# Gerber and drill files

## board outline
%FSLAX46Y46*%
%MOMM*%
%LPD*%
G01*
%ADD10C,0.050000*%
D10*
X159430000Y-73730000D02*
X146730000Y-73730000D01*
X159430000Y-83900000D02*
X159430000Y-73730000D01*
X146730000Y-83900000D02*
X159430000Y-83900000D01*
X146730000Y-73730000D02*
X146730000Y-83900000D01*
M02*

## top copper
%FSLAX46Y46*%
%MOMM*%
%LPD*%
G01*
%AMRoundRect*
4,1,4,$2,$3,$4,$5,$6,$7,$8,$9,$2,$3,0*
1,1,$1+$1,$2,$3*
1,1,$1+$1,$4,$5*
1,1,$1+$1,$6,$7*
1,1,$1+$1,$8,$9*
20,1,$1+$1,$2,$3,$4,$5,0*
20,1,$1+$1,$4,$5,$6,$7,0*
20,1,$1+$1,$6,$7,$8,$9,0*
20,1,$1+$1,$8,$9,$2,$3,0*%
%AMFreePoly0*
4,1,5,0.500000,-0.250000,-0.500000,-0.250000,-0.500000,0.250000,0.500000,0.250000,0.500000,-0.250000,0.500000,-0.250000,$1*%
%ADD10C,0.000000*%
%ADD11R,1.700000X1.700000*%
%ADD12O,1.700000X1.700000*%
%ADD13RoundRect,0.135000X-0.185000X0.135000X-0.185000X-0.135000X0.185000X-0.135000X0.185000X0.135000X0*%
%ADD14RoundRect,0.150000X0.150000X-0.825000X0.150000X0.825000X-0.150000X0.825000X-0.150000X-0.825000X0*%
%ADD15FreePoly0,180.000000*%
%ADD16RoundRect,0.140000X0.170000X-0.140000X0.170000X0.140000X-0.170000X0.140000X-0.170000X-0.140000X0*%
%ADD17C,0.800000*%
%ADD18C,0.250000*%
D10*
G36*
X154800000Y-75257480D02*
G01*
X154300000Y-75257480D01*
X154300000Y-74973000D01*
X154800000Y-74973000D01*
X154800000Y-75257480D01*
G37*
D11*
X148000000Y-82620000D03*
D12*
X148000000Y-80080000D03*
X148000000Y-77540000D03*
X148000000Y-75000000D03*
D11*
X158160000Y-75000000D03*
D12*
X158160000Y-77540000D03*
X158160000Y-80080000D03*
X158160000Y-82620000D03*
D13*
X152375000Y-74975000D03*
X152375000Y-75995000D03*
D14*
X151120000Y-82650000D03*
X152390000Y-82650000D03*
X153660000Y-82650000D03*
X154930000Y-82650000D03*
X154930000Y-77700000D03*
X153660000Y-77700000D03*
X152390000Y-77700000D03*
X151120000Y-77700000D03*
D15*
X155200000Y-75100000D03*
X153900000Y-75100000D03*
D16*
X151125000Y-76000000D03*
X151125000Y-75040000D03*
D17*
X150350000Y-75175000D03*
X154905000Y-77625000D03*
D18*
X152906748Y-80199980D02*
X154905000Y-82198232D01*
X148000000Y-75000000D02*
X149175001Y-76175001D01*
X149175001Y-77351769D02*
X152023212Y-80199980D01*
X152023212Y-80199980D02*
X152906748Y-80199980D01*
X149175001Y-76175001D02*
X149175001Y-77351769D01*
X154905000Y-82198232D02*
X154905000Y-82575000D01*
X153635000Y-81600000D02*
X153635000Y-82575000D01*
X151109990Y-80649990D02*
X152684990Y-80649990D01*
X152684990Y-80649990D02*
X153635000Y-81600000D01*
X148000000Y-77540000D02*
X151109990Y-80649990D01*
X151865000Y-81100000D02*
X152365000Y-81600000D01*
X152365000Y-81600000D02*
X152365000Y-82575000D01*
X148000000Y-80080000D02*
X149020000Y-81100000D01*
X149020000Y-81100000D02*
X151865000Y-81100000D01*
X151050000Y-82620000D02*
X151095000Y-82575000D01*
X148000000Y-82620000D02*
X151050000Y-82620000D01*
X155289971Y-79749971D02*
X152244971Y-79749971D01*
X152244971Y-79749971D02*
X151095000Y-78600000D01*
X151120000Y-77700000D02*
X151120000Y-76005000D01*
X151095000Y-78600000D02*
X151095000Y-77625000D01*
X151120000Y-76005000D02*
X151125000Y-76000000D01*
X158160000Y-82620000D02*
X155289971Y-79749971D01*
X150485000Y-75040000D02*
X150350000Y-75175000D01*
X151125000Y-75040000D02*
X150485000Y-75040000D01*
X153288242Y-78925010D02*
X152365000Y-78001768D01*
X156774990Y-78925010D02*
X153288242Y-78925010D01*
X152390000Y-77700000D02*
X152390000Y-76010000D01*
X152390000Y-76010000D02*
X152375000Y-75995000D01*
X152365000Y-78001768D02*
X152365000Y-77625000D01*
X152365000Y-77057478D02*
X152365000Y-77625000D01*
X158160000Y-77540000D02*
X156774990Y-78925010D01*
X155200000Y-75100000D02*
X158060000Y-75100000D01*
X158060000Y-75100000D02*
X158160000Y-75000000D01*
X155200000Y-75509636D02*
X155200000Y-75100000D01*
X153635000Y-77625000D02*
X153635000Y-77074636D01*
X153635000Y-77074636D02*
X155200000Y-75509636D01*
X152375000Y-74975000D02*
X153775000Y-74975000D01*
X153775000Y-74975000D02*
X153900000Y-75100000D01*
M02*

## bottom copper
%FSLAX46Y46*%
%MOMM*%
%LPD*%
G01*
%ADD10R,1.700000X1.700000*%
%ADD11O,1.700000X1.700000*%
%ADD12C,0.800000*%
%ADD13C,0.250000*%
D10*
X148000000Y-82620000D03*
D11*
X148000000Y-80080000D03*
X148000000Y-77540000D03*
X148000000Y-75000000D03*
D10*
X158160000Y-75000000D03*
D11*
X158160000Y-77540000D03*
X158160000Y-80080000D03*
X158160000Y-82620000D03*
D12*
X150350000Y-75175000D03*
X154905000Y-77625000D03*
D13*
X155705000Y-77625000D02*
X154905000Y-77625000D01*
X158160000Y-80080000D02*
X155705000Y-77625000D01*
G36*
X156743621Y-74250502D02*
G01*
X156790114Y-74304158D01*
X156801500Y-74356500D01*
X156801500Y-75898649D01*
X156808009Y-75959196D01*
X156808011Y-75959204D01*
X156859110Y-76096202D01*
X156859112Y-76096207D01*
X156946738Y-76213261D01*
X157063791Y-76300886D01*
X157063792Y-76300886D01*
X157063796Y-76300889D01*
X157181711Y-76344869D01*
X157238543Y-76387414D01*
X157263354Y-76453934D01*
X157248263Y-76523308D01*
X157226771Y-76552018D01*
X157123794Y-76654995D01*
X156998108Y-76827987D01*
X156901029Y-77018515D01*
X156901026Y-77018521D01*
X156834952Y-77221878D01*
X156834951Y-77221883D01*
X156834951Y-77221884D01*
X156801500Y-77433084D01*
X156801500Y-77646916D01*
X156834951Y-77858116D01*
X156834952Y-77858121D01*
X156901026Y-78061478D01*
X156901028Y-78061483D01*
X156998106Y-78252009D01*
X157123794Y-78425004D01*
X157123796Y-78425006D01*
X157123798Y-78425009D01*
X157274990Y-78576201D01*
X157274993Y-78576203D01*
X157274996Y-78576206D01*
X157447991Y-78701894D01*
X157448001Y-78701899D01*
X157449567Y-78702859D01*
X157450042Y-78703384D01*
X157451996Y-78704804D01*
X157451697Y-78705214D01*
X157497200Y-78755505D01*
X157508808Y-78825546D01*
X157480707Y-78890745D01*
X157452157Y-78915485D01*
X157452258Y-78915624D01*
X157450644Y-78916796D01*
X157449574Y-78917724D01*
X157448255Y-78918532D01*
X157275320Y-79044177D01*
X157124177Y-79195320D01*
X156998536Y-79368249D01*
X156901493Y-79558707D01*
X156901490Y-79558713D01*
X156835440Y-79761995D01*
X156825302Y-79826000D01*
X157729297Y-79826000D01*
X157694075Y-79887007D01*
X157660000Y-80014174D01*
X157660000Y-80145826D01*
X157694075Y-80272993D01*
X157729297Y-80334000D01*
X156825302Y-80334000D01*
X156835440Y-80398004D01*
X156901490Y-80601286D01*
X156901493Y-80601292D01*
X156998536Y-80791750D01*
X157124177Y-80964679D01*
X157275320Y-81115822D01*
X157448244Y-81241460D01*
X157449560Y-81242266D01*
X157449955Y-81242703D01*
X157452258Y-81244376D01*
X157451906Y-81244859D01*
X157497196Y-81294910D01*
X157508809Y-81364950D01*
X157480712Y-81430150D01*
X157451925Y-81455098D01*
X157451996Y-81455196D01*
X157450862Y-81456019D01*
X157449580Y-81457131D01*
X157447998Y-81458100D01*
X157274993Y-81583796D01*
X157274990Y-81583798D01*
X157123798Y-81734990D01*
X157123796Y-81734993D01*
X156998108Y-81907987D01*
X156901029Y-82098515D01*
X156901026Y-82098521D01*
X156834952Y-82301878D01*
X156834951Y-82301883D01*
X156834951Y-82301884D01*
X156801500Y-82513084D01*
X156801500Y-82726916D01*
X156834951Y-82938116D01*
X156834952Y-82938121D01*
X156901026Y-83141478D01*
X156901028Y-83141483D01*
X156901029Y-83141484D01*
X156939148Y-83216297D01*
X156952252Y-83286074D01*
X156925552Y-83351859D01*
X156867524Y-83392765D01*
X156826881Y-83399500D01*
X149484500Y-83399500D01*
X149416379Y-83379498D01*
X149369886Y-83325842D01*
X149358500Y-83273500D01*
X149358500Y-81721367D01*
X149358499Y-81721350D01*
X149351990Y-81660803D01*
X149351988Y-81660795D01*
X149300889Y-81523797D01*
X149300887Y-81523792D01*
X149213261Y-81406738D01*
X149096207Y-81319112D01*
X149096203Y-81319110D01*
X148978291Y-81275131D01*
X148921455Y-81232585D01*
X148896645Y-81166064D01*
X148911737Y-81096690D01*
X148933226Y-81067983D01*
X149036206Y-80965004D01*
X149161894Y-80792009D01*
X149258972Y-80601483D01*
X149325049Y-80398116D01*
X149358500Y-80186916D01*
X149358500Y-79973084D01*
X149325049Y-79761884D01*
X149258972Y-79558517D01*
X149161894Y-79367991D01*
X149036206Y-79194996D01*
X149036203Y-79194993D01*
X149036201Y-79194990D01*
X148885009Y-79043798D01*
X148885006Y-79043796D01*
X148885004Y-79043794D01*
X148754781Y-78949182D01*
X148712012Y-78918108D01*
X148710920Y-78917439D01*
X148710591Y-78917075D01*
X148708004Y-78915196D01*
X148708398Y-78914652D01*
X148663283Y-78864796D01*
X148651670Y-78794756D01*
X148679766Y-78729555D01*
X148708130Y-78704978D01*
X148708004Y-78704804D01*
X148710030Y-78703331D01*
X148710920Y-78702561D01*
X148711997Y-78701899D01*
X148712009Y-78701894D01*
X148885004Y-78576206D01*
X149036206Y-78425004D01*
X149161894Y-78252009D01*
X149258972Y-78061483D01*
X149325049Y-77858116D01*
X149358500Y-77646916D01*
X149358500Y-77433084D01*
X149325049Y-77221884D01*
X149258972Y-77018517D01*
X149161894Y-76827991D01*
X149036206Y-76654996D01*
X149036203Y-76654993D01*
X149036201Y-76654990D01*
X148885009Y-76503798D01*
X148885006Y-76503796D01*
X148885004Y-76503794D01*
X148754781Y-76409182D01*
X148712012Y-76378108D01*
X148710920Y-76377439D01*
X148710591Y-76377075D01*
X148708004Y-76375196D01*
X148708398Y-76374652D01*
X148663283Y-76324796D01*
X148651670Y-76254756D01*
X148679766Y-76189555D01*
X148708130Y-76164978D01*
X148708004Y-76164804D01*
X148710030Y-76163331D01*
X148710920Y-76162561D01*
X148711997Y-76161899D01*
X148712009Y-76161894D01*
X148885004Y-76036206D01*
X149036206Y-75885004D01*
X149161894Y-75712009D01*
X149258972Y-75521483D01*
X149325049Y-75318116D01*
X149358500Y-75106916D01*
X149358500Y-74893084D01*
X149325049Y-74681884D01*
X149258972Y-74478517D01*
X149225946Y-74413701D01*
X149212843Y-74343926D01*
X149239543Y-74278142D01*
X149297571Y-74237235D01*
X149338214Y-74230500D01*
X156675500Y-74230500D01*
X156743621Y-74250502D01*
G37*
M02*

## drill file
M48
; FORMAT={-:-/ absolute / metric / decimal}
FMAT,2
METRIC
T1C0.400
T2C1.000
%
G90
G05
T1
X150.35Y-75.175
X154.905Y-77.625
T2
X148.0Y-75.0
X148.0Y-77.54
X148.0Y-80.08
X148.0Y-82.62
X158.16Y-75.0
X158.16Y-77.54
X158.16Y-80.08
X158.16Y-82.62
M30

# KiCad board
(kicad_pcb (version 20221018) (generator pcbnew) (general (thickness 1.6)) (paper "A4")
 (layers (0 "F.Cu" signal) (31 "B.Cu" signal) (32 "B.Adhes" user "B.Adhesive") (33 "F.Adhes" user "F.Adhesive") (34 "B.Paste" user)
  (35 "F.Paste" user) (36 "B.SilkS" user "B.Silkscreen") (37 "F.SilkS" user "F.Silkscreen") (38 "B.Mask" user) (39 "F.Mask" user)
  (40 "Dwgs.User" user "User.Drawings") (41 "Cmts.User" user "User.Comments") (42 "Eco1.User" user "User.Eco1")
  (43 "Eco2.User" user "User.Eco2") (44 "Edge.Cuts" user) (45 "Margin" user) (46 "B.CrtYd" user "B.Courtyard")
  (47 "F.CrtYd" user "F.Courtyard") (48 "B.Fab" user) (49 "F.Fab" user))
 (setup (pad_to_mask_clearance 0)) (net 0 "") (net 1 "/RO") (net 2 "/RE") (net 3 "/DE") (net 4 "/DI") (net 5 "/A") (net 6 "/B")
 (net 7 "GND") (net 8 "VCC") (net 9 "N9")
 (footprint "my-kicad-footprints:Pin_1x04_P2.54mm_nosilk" (layer "F.Cu") (at 148 82.62 180)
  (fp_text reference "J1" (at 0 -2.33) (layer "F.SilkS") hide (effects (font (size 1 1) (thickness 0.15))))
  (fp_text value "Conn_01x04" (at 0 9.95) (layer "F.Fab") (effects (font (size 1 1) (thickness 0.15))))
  (pad "1" thru_hole rect (at 0 0 180) (size 1.7 1.7) (drill 1) (layers "*.Cu" "*.Mask") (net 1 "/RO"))
  (pad "2" thru_hole oval (at 0 2.54 180) (size 1.7 1.7) (drill 1) (layers "*.Cu" "*.Mask") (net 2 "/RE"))
  (pad "3" thru_hole oval (at 0 5.08 180) (size 1.7 1.7) (drill 1) (layers "*.Cu" "*.Mask") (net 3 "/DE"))
  (pad "4" thru_hole oval (at 0 7.62 180) (size 1.7 1.7) (drill 1) (layers "*.Cu" "*.Mask") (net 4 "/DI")))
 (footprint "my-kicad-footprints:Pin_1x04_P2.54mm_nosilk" (layer "F.Cu") (at 158.16 75)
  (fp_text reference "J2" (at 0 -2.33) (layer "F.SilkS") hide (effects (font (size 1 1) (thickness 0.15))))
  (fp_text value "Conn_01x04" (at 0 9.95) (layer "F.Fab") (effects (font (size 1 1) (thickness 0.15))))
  (pad "1" thru_hole rect (at 0 0) (size 1.7 1.7) (drill 1) (layers "*.Cu" "*.Mask") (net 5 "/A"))
  (pad "2" thru_hole oval (at 0 2.54) (size 1.7 1.7) (drill 1) (layers "*.Cu" "*.Mask") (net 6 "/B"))
  (pad "3" thru_hole oval (at 0 5.08) (size 1.7 1.7) (drill 1) (layers "*.Cu" "*.Mask") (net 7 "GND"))
  (pad "4" thru_hole oval (at 0 7.62) (size 1.7 1.7) (drill 1) (layers "*.Cu" "*.Mask") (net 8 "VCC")))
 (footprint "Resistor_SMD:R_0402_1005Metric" (layer "F.Cu") (at 152.375 75.485 -90)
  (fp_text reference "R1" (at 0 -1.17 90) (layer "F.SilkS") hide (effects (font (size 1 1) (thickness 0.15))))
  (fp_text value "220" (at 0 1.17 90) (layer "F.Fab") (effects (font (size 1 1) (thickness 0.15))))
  (pad "1" smd roundrect (at -0.51 0 270) (size 0.54 0.64) (layers "F.Cu" "F.Paste" "F.Mask") (roundrect_rratio 0.25) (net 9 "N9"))
  (pad "2" smd roundrect (at 0.51 0 270) (size 0.54 0.64) (layers "F.Cu" "F.Paste" "F.Mask") (roundrect_rratio 0.25) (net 6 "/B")))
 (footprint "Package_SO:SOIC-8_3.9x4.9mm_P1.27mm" (layer "F.Cu") (at 153.025 80.175 90)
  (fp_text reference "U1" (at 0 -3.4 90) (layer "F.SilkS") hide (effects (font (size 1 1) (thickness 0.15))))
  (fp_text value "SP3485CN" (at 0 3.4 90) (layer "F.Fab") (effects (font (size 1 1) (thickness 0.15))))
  (pad "1" smd roundrect (at -2.475 -1.905 90) (size 1.95 0.6) (layers "F.Cu" "F.Paste" "F.Mask") (roundrect_rratio 0.25) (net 1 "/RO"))
  (pad "2" smd roundrect (at -2.475 -0.635 90) (size 1.95 0.6) (layers "F.Cu" "F.Paste" "F.Mask") (roundrect_rratio 0.25) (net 2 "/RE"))
  (pad "3" smd roundrect (at -2.475 0.635 90) (size 1.95 0.6) (layers "F.Cu" "F.Paste" "F.Mask") (roundrect_rratio 0.25) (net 3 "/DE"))
  (pad "4" smd roundrect (at -2.475 1.905 90) (size 1.95 0.6) (layers "F.Cu" "F.Paste" "F.Mask") (roundrect_rratio 0.25) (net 4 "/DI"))
  (pad "5" smd roundrect (at 2.475 1.905 90) (size 1.95 0.6) (layers "F.Cu" "F.Paste" "F.Mask") (roundrect_rratio 0.25) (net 7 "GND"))
  (pad "6" smd roundrect (at 2.475 0.635 90) (size 1.95 0.6) (layers "F.Cu" "F.Paste" "F.Mask") (roundrect_rratio 0.25) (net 5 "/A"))
  (pad "7" smd roundrect (at 2.475 -0.635 90) (size 1.95 0.6) (layers "F.Cu" "F.Paste" "F.Mask") (roundrect_rratio 0.25) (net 6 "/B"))
  (pad "8" smd roundrect (at 2.475 -1.905 90) (size 1.95 0.6) (layers "F.Cu" "F.Paste" "F.Mask") (roundrect_rratio 0.25) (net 8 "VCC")))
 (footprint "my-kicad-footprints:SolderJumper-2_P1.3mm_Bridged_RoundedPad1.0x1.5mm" (layer "F.Cu") (at 154.55 75.1 180)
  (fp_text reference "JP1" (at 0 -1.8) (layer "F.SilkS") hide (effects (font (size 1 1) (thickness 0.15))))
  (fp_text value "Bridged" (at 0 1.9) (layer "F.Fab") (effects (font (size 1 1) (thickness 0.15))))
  (fp_poly
   (pts (xy 0.25 -0.15748) (xy -0.25 -0.15748) (xy -0.25 0.127) (xy 0.25 0.127)) (stroke (width 0) (type solid)) (fill solid) (layer "F.Cu"))
  (pad "1" smd custom (at -0.65 0 180) (size 1 0.5) (layers "F.Cu" "F.Mask") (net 5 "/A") (zone_connect 2) (thermal_bridge_angle 45)
   (options (clearance outline) (anchor rect)) (primitives))
  (pad "2" smd custom (at 0.65 0 180) (size 1 0.5) (layers "F.Cu" "F.Mask") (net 9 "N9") (zone_connect 2) (thermal_bridge_angle 45)
   (options (clearance outline) (anchor rect)) (primitives)))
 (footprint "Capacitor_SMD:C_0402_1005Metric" (layer "F.Cu") (at 151.125 75.52 90)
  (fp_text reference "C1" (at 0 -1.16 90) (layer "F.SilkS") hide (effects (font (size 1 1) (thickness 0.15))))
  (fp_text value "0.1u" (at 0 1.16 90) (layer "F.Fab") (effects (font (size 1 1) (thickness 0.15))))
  (pad "1" smd roundrect (at -0.48 0 90) (size 0.56 0.62) (layers "F.Cu" "F.Paste" "F.Mask") (roundrect_rratio 0.25) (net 8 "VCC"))
  (pad "2" smd roundrect (at 0.48 0 90) (size 0.56 0.62) (layers "F.Cu" "F.Paste" "F.Mask") (roundrect_rratio 0.25) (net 7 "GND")))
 (gr_line (start 159.43 73.73) (end 146.73 73.73) (stroke (width 0.05) (type solid)) (layer "Edge.Cuts"))
 (gr_line (start 159.43 83.9) (end 159.43 73.73) (stroke (width 0.05) (type solid)) (layer "Edge.Cuts"))
 (gr_line (start 146.73 83.9) (end 159.43 83.9) (stroke (width 0.05) (type solid)) (layer "Edge.Cuts"))
 (gr_line (start 146.73 73.73) (end 146.73 83.9) (stroke (width 0.05) (type solid)) (layer "Edge.Cuts"))
 (segment (start 152.906748 80.19998) (end 154.905 82.198232) (width 0.25) (layer "F.Cu") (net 4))
 (segment (start 148 75) (end 149.175001 76.175001) (width 0.25) (layer "F.Cu") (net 4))
 (segment (start 149.175001 77.351769) (end 152.023212 80.19998) (width 0.25) (layer "F.Cu") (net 4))
 (segment (start 152.023212 80.19998) (end 152.906748 80.19998) (width 0.25) (layer "F.Cu") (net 4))
 (segment (start 149.175001 76.175001) (end 149.175001 77.351769) (width 0.25) (layer "F.Cu") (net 4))
 (segment (start 154.905 82.198232) (end 154.905 82.575) (width 0.25) (layer "F.Cu") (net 4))
 (segment (start 153.635 81.6) (end 153.635 82.575) (width 0.25) (layer "F.Cu") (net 3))
 (segment (start 151.10999 80.64999) (end 152.68499 80.64999) (width 0.25) (layer "F.Cu") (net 3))
 (segment (start 152.68499 80.64999) (end 153.635 81.6) (width 0.25) (layer "F.Cu") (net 3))
 (segment (start 148 77.54) (end 151.10999 80.64999) (width 0.25) (layer "F.Cu") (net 3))
 (segment (start 151.865 81.1) (end 152.365 81.6) (width 0.25) (layer "F.Cu") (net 2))
 (segment (start 152.365 81.6) (end 152.365 82.575) (width 0.25) (layer "F.Cu") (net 2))
 (segment (start 148 80.08) (end 149.02 81.1) (width 0.25) (layer "F.Cu") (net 2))
 (segment (start 149.02 81.1) (end 151.865 81.1) (width 0.25) (layer "F.Cu") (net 2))
 (segment (start 151.05 82.62) (end 151.095 82.575) (width 0.25) (layer "F.Cu") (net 1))
 (segment (start 148 82.62) (end 151.05 82.62) (width 0.25) (layer "F.Cu") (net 1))
 (segment (start 155.289971 79.749971) (end 152.244971 79.749971) (width 0.25) (layer "F.Cu") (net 8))
 (segment (start 152.244971 79.749971) (end 151.095 78.6) (width 0.25) (layer "F.Cu") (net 8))
 (segment (start 151.12 77.7) (end 151.12 76.005) (width 0.25) (layer "F.Cu") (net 8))
 (segment (start 151.095 78.6) (end 151.095 77.625) (width 0.25) (layer "F.Cu") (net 8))
 (segment (start 151.12 76.005) (end 151.125 76) (width 0.25) (layer "F.Cu") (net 8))
 (segment (start 158.16 82.62) (end 155.289971 79.749971) (width 0.25) (layer "F.Cu") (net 8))
 (segment (start 150.485 75.04) (end 150.35 75.175) (width 0.25) (layer "F.Cu") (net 7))
 (segment (start 151.125 75.04) (end 150.485 75.04) (width 0.25) (layer "F.Cu") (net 7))
 (via (at 150.35 75.175) (size 0.8) (drill 0.4) (layers "F.Cu" "B.Cu") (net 7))
 (via (at 154.905 77.625) (size 0.8) (drill 0.4) (layers "F.Cu" "B.Cu") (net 7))
 (segment (start 155.705 77.625) (end 154.905 77.625) (width 0.25) (layer "B.Cu") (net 7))
 (segment (start 158.16 80.08) (end 155.705 77.625) (width 0.25) (layer "B.Cu") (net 7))
 (segment (start 153.288242 78.92501) (end 152.365 78.001768) (width 0.25) (layer "F.Cu") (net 6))
 (segment (start 156.77499 78.92501) (end 153.288242 78.92501) (width 0.25) (layer "F.Cu") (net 6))
 (segment (start 152.39 77.7) (end 152.39 76.01) (width 0.25) (layer "F.Cu") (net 6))
 (segment (start 152.39 76.01) (end 152.375 75.995) (width 0.25) (layer "F.Cu") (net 6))
 (segment (start 152.365 78.001768) (end 152.365 77.625) (width 0.25) (layer "F.Cu") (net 6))
 (segment (start 152.365 77.057478) (end 152.365 77.625) (width 0.25) (layer "F.Cu") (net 6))
 (segment (start 158.16 77.54) (end 156.77499 78.92501) (width 0.25) (layer "F.Cu") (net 6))
 (segment (start 155.2 75.1) (end 158.06 75.1) (width 0.25) (layer "F.Cu") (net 5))
 (segment (start 158.06 75.1) (end 158.16 75) (width 0.25) (layer "F.Cu") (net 5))
 (segment (start 155.2 75.509636) (end 155.2 75.1) (width 0.25) (layer "F.Cu") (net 5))
 (segment (start 153.635 77.625) (end 153.635 77.074636) (width 0.25) (layer "F.Cu") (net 5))
 (segment (start 153.635 77.074636) (end 155.2 75.509636) (width 0.25) (layer "F.Cu") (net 5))
 (segment (start 152.375 74.975) (end 153.775 74.975) (width 0.25) (layer "F.Cu") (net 9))
 (segment (start 153.775 74.975) (end 153.9 75.1) (width 0.25) (layer "F.Cu") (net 9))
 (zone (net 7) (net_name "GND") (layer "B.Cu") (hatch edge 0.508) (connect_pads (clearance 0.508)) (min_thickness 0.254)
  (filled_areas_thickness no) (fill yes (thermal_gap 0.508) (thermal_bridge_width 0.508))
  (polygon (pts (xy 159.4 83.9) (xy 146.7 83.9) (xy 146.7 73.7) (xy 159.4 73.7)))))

